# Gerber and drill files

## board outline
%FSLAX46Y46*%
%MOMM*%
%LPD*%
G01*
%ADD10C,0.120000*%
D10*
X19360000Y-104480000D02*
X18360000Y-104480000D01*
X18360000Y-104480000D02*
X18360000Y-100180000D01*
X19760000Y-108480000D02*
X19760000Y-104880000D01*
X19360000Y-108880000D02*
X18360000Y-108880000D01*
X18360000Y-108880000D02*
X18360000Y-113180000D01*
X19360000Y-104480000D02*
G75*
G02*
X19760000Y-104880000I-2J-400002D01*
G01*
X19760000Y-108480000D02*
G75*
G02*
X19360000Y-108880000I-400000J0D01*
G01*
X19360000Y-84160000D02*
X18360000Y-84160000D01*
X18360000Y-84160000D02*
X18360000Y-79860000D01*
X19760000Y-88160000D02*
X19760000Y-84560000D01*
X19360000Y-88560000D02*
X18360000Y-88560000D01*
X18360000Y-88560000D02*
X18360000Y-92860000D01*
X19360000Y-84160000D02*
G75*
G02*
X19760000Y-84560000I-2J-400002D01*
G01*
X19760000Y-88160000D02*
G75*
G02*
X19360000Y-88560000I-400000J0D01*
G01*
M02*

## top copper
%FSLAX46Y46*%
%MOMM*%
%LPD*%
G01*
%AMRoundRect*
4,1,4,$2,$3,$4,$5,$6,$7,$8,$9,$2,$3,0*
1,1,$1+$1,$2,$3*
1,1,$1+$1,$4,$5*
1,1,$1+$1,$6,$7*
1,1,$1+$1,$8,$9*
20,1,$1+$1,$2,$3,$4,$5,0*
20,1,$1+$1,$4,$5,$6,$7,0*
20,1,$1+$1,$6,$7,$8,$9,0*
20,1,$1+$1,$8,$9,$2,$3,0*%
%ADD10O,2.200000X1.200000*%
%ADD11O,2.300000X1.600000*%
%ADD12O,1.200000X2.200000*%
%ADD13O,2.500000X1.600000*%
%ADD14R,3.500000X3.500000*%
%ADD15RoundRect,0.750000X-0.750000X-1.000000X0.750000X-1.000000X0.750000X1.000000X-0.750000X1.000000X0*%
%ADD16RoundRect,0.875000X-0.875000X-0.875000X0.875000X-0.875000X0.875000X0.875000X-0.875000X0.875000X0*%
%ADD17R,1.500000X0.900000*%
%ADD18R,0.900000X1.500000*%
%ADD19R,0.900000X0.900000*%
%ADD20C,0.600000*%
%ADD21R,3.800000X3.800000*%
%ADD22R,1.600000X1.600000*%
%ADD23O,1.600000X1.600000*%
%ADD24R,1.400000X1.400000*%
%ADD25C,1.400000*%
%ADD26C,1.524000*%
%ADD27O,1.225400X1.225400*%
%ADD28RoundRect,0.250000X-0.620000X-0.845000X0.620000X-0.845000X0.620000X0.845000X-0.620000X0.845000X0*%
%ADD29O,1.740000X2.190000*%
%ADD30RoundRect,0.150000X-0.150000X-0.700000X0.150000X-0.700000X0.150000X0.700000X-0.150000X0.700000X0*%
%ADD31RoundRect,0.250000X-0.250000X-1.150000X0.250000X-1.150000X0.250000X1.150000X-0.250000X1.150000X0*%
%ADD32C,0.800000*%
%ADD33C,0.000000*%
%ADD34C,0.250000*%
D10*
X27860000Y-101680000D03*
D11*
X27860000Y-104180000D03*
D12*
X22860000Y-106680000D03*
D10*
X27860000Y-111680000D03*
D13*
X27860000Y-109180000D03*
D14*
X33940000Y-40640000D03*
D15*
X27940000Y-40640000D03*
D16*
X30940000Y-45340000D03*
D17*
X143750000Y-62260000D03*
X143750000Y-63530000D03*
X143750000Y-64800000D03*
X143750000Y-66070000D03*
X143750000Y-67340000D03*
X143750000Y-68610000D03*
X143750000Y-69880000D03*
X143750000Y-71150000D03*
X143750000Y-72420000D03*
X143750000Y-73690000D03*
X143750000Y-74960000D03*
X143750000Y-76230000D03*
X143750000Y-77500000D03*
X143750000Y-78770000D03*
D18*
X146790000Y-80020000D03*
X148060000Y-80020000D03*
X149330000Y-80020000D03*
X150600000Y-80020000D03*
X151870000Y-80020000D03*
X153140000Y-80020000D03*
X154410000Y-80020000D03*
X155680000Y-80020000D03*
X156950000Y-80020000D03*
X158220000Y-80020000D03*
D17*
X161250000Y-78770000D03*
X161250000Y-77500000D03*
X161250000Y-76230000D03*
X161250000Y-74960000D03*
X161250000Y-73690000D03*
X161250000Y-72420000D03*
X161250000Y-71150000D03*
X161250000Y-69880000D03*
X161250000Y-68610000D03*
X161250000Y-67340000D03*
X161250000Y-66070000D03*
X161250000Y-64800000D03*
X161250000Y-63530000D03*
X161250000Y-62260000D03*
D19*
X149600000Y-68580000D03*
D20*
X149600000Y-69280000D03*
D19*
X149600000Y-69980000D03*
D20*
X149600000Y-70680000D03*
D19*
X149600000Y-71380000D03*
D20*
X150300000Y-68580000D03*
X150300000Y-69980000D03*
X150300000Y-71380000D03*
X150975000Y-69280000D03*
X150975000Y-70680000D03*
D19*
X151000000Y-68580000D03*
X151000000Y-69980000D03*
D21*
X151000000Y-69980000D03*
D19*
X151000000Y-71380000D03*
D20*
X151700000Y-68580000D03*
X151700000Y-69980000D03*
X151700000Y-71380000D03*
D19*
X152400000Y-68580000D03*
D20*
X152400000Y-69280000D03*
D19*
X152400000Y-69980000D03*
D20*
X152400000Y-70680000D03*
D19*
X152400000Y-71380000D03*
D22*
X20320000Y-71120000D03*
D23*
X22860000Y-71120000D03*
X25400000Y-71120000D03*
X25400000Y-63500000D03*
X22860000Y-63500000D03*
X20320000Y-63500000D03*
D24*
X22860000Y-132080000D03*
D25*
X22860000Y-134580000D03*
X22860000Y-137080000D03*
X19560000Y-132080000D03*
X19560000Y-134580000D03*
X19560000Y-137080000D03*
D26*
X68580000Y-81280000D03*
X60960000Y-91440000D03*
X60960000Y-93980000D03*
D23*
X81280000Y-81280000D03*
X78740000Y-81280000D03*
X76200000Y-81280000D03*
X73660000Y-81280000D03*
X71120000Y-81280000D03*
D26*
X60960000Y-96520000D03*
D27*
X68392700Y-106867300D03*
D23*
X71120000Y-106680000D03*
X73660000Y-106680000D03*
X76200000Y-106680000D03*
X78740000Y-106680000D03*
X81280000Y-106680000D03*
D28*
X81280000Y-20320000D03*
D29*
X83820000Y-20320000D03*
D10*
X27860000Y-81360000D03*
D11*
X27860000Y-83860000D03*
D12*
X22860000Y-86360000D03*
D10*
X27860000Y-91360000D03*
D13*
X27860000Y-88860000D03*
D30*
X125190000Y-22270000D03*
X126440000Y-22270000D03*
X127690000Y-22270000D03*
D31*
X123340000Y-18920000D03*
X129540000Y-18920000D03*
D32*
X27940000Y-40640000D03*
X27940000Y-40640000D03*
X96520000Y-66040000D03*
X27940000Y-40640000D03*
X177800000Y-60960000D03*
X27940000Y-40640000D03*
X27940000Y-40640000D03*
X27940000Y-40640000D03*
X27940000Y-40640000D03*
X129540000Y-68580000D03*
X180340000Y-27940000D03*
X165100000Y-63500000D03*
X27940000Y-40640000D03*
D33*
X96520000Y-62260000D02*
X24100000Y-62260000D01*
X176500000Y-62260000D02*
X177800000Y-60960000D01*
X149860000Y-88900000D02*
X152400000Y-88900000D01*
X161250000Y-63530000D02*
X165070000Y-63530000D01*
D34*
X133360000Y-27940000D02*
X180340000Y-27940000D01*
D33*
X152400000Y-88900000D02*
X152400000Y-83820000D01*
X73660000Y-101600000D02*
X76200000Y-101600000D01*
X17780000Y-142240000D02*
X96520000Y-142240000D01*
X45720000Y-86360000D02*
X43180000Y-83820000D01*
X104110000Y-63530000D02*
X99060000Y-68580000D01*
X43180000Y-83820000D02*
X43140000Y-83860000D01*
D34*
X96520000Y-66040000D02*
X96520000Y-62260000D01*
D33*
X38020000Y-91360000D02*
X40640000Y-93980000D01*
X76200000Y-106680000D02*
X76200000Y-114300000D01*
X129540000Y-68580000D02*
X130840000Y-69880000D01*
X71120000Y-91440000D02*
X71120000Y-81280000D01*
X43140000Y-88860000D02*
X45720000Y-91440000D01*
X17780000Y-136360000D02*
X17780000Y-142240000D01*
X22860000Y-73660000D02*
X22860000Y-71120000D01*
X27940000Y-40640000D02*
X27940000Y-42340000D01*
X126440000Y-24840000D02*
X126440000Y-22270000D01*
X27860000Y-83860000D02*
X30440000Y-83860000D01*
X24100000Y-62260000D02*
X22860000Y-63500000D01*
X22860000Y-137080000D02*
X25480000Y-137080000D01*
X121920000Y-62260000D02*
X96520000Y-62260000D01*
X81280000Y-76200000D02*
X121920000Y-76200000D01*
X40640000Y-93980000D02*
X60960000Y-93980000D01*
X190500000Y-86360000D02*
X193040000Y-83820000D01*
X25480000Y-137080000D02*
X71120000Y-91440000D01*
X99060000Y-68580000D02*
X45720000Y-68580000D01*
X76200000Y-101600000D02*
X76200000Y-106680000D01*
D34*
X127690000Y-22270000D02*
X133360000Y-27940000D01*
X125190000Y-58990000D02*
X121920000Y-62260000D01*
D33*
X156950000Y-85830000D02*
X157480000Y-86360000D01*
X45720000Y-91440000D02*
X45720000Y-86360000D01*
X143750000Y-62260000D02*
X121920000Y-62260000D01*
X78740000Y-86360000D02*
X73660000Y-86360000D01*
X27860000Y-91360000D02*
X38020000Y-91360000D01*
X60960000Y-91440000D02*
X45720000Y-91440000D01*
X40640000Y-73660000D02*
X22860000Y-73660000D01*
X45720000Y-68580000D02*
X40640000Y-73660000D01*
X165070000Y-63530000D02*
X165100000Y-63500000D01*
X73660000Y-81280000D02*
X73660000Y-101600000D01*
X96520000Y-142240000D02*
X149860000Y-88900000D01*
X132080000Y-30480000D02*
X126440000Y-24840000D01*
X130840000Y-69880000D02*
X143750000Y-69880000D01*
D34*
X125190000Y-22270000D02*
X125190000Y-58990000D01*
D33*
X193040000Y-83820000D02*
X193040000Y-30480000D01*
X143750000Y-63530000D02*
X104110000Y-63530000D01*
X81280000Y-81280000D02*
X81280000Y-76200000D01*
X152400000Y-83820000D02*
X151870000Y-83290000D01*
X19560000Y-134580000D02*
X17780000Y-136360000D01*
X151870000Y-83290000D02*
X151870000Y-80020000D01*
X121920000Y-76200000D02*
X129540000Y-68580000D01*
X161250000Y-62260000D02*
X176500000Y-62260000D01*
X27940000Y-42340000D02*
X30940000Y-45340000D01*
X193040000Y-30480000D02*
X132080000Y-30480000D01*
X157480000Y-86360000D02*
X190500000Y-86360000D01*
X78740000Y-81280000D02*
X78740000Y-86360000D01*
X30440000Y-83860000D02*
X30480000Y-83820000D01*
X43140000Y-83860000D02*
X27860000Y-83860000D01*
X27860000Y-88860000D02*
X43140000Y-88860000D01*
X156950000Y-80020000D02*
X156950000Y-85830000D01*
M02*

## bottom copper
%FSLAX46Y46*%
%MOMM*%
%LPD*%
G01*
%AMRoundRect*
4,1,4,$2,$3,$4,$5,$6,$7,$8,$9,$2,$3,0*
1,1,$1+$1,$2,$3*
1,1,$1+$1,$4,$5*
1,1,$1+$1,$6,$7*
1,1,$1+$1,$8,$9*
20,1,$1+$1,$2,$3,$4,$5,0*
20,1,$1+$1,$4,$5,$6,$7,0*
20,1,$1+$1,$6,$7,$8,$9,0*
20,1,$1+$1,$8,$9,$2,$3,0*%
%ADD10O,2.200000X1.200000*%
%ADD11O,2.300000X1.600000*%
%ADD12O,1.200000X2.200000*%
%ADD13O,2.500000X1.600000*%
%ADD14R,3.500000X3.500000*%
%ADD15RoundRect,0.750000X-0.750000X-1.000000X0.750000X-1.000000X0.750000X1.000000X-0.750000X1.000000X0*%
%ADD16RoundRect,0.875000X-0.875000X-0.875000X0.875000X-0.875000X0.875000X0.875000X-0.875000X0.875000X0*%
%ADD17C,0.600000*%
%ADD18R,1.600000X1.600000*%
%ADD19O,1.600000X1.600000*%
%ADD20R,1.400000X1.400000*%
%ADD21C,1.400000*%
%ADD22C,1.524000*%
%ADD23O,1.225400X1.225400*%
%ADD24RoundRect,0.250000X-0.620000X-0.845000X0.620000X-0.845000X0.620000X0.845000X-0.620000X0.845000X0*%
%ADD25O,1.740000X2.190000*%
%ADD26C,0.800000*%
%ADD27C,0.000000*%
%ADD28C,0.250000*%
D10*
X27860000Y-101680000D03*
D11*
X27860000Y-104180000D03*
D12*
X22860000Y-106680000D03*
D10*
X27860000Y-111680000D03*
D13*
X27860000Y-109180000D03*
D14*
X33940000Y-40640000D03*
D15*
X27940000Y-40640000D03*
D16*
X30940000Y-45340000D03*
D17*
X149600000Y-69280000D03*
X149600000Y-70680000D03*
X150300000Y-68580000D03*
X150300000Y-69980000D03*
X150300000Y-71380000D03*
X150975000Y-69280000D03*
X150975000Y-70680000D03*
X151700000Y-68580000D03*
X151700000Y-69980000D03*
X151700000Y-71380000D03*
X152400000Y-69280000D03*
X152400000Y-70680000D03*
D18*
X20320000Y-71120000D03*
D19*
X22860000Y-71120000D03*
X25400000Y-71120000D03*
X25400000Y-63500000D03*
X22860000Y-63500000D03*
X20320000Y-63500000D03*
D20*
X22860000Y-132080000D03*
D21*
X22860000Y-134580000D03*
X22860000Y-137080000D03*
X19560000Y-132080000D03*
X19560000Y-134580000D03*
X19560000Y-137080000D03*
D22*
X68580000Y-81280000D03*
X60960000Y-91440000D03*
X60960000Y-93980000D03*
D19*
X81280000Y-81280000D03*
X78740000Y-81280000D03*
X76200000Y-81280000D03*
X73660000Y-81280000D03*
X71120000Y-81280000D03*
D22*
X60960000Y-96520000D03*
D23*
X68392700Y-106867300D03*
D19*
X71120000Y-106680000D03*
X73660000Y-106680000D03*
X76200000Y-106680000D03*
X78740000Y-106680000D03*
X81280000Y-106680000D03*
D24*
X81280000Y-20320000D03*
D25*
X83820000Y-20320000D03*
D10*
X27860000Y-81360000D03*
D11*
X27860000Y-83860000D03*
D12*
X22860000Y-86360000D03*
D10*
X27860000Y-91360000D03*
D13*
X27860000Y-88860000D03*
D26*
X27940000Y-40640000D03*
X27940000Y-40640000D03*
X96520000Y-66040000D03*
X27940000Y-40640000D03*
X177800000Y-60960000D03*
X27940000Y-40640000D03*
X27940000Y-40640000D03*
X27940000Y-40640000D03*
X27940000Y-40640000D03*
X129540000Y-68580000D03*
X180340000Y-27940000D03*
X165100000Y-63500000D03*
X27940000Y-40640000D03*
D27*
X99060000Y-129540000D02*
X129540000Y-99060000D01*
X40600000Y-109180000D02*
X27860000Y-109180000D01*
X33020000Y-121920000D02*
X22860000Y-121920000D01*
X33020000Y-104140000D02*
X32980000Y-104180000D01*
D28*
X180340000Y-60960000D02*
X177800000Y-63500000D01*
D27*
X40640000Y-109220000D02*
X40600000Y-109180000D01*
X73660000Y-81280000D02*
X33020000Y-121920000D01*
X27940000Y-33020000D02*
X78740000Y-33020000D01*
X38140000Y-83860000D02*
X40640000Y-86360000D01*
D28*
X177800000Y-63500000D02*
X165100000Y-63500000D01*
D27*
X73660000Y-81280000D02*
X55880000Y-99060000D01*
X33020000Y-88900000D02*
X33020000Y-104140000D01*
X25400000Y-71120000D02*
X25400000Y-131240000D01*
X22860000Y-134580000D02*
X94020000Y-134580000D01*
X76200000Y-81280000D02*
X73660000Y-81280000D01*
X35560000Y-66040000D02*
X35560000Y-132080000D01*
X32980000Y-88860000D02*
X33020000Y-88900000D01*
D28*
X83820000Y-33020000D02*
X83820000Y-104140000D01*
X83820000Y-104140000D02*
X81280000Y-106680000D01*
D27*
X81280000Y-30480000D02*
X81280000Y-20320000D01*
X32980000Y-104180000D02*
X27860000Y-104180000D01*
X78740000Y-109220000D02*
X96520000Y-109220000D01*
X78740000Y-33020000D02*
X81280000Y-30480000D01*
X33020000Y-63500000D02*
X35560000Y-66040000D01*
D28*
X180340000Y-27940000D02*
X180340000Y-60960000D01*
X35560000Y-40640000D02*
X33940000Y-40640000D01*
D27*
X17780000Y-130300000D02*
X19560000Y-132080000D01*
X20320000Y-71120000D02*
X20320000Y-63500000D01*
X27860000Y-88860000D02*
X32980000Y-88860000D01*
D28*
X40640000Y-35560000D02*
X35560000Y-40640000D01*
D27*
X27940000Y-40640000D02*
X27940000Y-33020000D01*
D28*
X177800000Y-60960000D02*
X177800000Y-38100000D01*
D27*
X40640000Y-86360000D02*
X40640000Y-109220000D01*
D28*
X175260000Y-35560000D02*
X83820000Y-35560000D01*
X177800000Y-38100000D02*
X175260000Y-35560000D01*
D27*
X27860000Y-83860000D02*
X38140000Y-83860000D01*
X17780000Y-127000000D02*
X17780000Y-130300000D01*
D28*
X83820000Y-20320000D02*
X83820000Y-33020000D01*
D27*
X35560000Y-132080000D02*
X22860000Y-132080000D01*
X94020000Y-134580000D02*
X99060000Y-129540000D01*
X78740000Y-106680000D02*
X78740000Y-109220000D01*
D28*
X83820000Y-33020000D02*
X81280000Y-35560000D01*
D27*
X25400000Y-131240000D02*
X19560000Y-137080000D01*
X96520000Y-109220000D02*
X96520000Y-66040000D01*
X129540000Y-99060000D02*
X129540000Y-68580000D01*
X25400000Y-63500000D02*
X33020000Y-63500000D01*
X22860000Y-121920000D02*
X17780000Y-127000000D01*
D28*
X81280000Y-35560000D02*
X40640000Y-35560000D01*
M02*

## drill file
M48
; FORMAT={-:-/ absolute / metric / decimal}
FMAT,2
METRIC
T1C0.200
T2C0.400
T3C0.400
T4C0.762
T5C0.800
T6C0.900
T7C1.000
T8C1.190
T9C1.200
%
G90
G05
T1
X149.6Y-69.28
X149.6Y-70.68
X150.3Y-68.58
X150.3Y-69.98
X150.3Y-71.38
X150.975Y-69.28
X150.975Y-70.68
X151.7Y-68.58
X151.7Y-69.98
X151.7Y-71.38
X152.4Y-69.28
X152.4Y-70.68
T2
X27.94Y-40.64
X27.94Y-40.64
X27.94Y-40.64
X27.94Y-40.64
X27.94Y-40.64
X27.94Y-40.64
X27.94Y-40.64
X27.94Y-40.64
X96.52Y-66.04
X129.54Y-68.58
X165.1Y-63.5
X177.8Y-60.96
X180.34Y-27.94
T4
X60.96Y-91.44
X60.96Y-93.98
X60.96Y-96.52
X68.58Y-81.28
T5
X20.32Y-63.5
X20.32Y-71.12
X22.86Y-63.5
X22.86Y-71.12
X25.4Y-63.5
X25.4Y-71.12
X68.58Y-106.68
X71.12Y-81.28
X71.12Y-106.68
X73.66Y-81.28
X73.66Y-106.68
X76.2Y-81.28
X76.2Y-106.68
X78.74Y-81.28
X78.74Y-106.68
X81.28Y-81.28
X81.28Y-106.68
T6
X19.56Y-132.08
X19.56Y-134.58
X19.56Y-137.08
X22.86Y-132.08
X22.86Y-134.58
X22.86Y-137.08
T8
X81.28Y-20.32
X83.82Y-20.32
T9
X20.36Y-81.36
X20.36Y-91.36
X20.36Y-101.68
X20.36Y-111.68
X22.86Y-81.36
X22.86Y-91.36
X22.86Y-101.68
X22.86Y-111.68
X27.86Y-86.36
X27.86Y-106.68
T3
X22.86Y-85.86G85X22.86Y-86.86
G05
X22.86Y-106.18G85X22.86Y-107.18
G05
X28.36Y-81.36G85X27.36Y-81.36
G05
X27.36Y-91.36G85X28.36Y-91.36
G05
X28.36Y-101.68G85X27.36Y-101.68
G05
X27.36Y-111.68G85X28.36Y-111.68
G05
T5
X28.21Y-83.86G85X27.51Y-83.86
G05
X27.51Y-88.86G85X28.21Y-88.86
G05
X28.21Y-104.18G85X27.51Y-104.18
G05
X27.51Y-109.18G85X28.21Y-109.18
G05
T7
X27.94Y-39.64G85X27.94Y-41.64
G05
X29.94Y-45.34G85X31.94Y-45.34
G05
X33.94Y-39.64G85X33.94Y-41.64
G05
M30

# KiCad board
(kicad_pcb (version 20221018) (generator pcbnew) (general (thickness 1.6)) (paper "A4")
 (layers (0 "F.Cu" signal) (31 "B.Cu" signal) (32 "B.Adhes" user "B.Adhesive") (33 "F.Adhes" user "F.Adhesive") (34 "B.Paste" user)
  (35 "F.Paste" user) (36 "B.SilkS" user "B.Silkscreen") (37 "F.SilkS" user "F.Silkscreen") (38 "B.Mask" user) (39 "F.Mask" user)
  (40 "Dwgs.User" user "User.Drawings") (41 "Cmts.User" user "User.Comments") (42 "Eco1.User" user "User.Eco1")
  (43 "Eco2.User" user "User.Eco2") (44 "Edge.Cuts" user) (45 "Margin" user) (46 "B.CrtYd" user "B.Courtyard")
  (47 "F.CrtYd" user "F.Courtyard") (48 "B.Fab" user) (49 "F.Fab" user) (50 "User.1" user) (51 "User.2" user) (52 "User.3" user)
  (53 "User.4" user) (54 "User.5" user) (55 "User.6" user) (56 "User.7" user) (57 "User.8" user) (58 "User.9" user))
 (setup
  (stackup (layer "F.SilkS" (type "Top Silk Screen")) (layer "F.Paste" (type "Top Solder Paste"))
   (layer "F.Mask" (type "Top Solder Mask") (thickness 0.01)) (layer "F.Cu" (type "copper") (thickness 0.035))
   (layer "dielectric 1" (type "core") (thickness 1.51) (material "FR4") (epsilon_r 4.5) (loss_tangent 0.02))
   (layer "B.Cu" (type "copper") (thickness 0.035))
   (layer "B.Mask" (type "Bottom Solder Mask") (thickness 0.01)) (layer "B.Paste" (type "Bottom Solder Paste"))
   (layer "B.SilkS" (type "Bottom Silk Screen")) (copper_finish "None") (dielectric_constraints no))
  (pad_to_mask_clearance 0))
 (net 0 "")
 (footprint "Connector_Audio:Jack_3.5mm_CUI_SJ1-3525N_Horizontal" (layer "F.Cu") (at 22.86 106.68 -90)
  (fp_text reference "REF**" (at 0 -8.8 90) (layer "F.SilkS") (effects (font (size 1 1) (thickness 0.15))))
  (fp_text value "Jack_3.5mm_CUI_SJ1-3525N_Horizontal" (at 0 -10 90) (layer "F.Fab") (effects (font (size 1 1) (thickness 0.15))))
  (fp_line (start -2.2 3.5) (end -2.2 4.5) (stroke (width 0.12) (type solid)) (layer "Edge.Cuts"))
  (fp_line (start -2.2 4.5) (end -6.5 4.5) (stroke (width 0.12) (type solid)) (layer "Edge.Cuts"))
  (fp_line (start 1.8 3.1) (end -1.8 3.1) (stroke (width 0.12) (type solid)) (layer "Edge.Cuts"))
  (fp_line (start 2.2 3.5) (end 2.2 4.5) (stroke (width 0.12) (type solid)) (layer "Edge.Cuts"))
  (fp_line (start 2.2 4.5) (end 6.5 4.5) (stroke (width 0.12) (type solid)) (layer "Edge.Cuts"))
  (fp_arc (start -2.2 3.5) (mid -2.082842 3.217158) (end -1.8 3.1) (stroke (width 0.12) (type solid)) (layer "Edge.Cuts"))
  (fp_arc (start 1.8 3.1) (mid 2.082843 3.217157) (end 2.2 3.5) (stroke (width 0.12) (type solid)) (layer "Edge.Cuts"))
  (pad "" np_thru_hole circle (at -5 0 270) (size 1.2 1.2) (drill 1.2) (layers "*.Cu"))
  (pad "" np_thru_hole circle (at -5 2.5 270) (size 1.2 1.2) (drill 1.2) (layers "*.Cu"))
  (pad "" np_thru_hole circle (at 0 -5 270) (size 1.2 1.2) (drill 1.2) (layers "*.Cu"))
  (pad "" np_thru_hole circle (at 5 0 270) (size 1.2 1.2) (drill 1.2) (layers "*.Cu"))
  (pad "" np_thru_hole circle (at 5 2.5 270) (size 1.2 1.2) (drill 1.2) (layers "*.Cu"))
  (pad "R" thru_hole oval (at -5 -5 270) (size 1.2 2.2) (drill oval 0.4 1.4) (layers "*.Cu" "*.Mask"))
  (pad "RN" thru_hole oval (at -2.5 -5 270) (size 1.6 2.3) (drill oval 0.8 1.5) (layers "*.Cu" "*.Mask"))
  (pad "S" thru_hole oval (at 0 0 270) (size 2.2 1.2) (drill oval 1.4 0.4) (layers "*.Cu" "*.Mask"))
  (pad "T" thru_hole oval (at 5 -5 90) (size 1.2 2.2) (drill oval 0.4 1.4) (layers "*.Cu" "*.Mask"))
  (pad "TN" thru_hole oval (at 2.5 -5 90) (size 1.6 2.5) (drill oval 0.8 1.5) (layers "*.Cu" "*.Mask")))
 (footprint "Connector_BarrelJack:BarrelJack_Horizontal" (layer "F.Cu") (at 33.94 40.64)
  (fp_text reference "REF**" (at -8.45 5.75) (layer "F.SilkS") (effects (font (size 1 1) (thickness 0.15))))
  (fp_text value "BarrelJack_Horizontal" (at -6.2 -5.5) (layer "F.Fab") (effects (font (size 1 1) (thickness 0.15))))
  (pad "1" thru_hole rect (at 0 0) (size 3.5 3.5) (drill oval 1 3) (layers "*.Cu" "*.Mask"))
  (pad "2" thru_hole roundrect (at -6 0) (size 3 3.5) (drill oval 1 3) (layers "*.Cu" "*.Mask") (roundrect_rratio 0.25))
  (pad "3" thru_hole roundrect (at -3 4.7) (size 3.5 3.5) (drill oval 3 1) (layers "*.Cu" "*.Mask") (roundrect_rratio 0.25)))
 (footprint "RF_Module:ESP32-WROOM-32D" (layer "F.Cu") (at 152.5 70.51)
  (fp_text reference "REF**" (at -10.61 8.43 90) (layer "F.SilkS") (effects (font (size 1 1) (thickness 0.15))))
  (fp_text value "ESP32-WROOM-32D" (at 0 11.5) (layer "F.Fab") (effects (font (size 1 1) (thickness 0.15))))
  (pad "1" smd rect (at -8.75 -8.25) (size 1.5 0.9) (layers "F.Cu" "F.Paste" "F.Mask"))
  (pad "2" smd rect (at -8.75 -6.98) (size 1.5 0.9) (layers "F.Cu" "F.Paste" "F.Mask"))
  (pad "3" smd rect (at -8.75 -5.71) (size 1.5 0.9) (layers "F.Cu" "F.Paste" "F.Mask"))
  (pad "4" smd rect (at -8.75 -4.44) (size 1.5 0.9) (layers "F.Cu" "F.Paste" "F.Mask"))
  (pad "5" smd rect (at -8.75 -3.17) (size 1.5 0.9) (layers "F.Cu" "F.Paste" "F.Mask"))
  (pad "6" smd rect (at -8.75 -1.9) (size 1.5 0.9) (layers "F.Cu" "F.Paste" "F.Mask"))
  (pad "7" smd rect (at -8.75 -0.63) (size 1.5 0.9) (layers "F.Cu" "F.Paste" "F.Mask"))
  (pad "8" smd rect (at -8.75 0.64) (size 1.5 0.9) (layers "F.Cu" "F.Paste" "F.Mask"))
  (pad "9" smd rect (at -8.75 1.91) (size 1.5 0.9) (layers "F.Cu" "F.Paste" "F.Mask"))
  (pad "10" smd rect (at -8.75 3.18) (size 1.5 0.9) (layers "F.Cu" "F.Paste" "F.Mask"))
  (pad "11" smd rect (at -8.75 4.45) (size 1.5 0.9) (layers "F.Cu" "F.Paste" "F.Mask"))
  (pad "12" smd rect (at -8.75 5.72) (size 1.5 0.9) (layers "F.Cu" "F.Paste" "F.Mask"))
  (pad "13" smd rect (at -8.75 6.99) (size 1.5 0.9) (layers "F.Cu" "F.Paste" "F.Mask"))
  (pad "14" smd rect (at -8.75 8.26) (size 1.5 0.9) (layers "F.Cu" "F.Paste" "F.Mask"))
  (pad "15" smd rect (at -5.71 9.51 90) (size 1.5 0.9) (layers "F.Cu" "F.Paste" "F.Mask"))
  (pad "16" smd rect (at -4.44 9.51 90) (size 1.5 0.9) (layers "F.Cu" "F.Paste" "F.Mask"))
  (pad "17" smd rect (at -3.17 9.51 90) (size 1.5 0.9) (layers "F.Cu" "F.Paste" "F.Mask"))
  (pad "18" smd rect (at -1.9 9.51 90) (size 1.5 0.9) (layers "F.Cu" "F.Paste" "F.Mask"))
  (pad "19" smd rect (at -0.63 9.51 90) (size 1.5 0.9) (layers "F.Cu" "F.Paste" "F.Mask"))
  (pad "20" smd rect (at 0.64 9.51 90) (size 1.5 0.9) (layers "F.Cu" "F.Paste" "F.Mask"))
  (pad "21" smd rect (at 1.91 9.51 90) (size 1.5 0.9) (layers "F.Cu" "F.Paste" "F.Mask"))
  (pad "22" smd rect (at 3.18 9.51 90) (size 1.5 0.9) (layers "F.Cu" "F.Paste" "F.Mask"))
  (pad "23" smd rect (at 4.45 9.51 90) (size 1.5 0.9) (layers "F.Cu" "F.Paste" "F.Mask"))
  (pad "24" smd rect (at 5.72 9.51 90) (size 1.5 0.9) (layers "F.Cu" "F.Paste" "F.Mask"))
  (pad "25" smd rect (at 8.75 8.26) (size 1.5 0.9) (layers "F.Cu" "F.Paste" "F.Mask"))
  (pad "26" smd rect (at 8.75 6.99) (size 1.5 0.9) (layers "F.Cu" "F.Paste" "F.Mask"))
  (pad "27" smd rect (at 8.75 5.72) (size 1.5 0.9) (layers "F.Cu" "F.Paste" "F.Mask"))
  (pad "28" smd rect (at 8.75 4.45) (size 1.5 0.9) (layers "F.Cu" "F.Paste" "F.Mask"))
  (pad "29" smd rect (at 8.75 3.18) (size 1.5 0.9) (layers "F.Cu" "F.Paste" "F.Mask"))
  (pad "30" smd rect (at 8.75 1.91) (size 1.5 0.9) (layers "F.Cu" "F.Paste" "F.Mask"))
  (pad "31" smd rect (at 8.75 0.64) (size 1.5 0.9) (layers "F.Cu" "F.Paste" "F.Mask"))
  (pad "32" smd rect (at 8.75 -0.63) (size 1.5 0.9) (layers "F.Cu" "F.Paste" "F.Mask"))
  (pad "33" smd rect (at 8.75 -1.9) (size 1.5 0.9) (layers "F.Cu" "F.Paste" "F.Mask"))
  (pad "34" smd rect (at 8.75 -3.17) (size 1.5 0.9) (layers "F.Cu" "F.Paste" "F.Mask"))
  (pad "35" smd rect (at 8.75 -4.44) (size 1.5 0.9) (layers "F.Cu" "F.Paste" "F.Mask"))
  (pad "36" smd rect (at 8.75 -5.71) (size 1.5 0.9) (layers "F.Cu" "F.Paste" "F.Mask"))
  (pad "37" smd rect (at 8.75 -6.98) (size 1.5 0.9) (layers "F.Cu" "F.Paste" "F.Mask"))
  (pad "38" smd rect (at 8.75 -8.25) (size 1.5 0.9) (layers "F.Cu" "F.Paste" "F.Mask"))
  (pad "39" smd rect (at -2.9 -1.93) (size 0.9 0.9) (layers "F.Cu" "F.Paste"))
  (pad "39" thru_hole circle (at -2.9 -1.23) (size 0.6 0.6) (drill 0.2) (layers "*.Cu" "F.Mask"))
  (pad "39" smd rect (at -2.9 -0.53) (size 0.9 0.9) (layers "F.Cu" "F.Paste"))
  (pad "39" thru_hole circle (at -2.9 0.17) (size 0.6 0.6) (drill 0.2) (layers "*.Cu" "F.Mask"))
  (pad "39" smd rect (at -2.9 0.87) (size 0.9 0.9) (layers "F.Cu" "F.Paste"))
  (pad "39" thru_hole circle (at -2.2 -1.93) (size 0.6 0.6) (drill 0.2) (layers "*.Cu" "F.Mask"))
  (pad "39" thru_hole circle (at -2.2 -0.53) (size 0.6 0.6) (drill 0.2) (layers "*.Cu" "F.Mask"))
  (pad "39" thru_hole circle (at -2.2 0.87) (size 0.6 0.6) (drill 0.2) (layers "*.Cu" "F.Mask"))
  (pad "39" thru_hole circle (at -1.525 -1.23) (size 0.6 0.6) (drill 0.2) (layers "*.Cu" "F.Mask"))
  (pad "39" thru_hole circle (at -1.525 0.17) (size 0.6 0.6) (drill 0.2) (layers "*.Cu" "F.Mask"))
  (pad "39" smd rect (at -1.5 -1.93) (size 0.9 0.9) (layers "F.Cu" "F.Paste"))
  (pad "39" smd rect (at -1.5 -0.53) (size 0.9 0.9) (layers "F.Cu" "F.Paste"))
  (pad "39" smd rect (at -1.5 -0.53) (size 3.8 3.8) (layers "F.Cu" "F.Mask"))
  (pad "39" smd rect (at -1.5 0.87) (size 0.9 0.9) (layers "F.Cu" "F.Paste"))
  (pad "39" thru_hole circle (at -0.8 -1.93) (size 0.6 0.6) (drill 0.2) (layers "*.Cu" "F.Mask"))
  (pad "39" thru_hole circle (at -0.8 -0.53) (size 0.6 0.6) (drill 0.2) (layers "*.Cu" "F.Mask"))
  (pad "39" thru_hole circle (at -0.8 0.87) (size 0.6 0.6) (drill 0.2) (layers "*.Cu" "F.Mask"))
  (pad "39" smd rect (at -0.1 -1.93) (size 0.9 0.9) (layers "F.Cu" "F.Paste"))
  (pad "39" thru_hole circle (at -0.1 -1.23) (size 0.6 0.6) (drill 0.2) (layers "*.Cu" "F.Mask"))
  (pad "39" smd rect (at -0.1 -0.53) (size 0.9 0.9) (layers "F.Cu" "F.Paste"))
  (pad "39" thru_hole circle (at -0.1 0.17) (size 0.6 0.6) (drill 0.2) (layers "*.Cu" "F.Mask"))
  (pad "39" smd rect (at -0.1 0.87) (size 0.9 0.9) (layers "F.Cu" "F.Paste"))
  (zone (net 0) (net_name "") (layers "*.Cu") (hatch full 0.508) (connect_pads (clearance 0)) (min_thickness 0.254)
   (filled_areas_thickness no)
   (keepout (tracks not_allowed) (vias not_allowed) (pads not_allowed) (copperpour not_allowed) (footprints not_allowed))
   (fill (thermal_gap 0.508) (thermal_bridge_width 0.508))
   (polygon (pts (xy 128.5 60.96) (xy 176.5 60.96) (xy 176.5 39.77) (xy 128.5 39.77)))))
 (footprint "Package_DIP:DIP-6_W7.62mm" (layer "F.Cu") (at 20.32 71.12 90)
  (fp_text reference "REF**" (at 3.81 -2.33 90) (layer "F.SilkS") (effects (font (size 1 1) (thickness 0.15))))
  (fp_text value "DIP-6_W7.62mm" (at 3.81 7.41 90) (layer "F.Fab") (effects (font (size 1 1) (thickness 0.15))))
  (pad "1" thru_hole rect (at 0 0 90) (size 1.6 1.6) (drill 0.8) (layers "*.Cu" "*.Mask"))
  (pad "2" thru_hole oval (at 0 2.54 90) (size 1.6 1.6) (drill 0.8) (layers "*.Cu" "*.Mask"))
  (pad "3" thru_hole oval (at 0 5.08 90) (size 1.6 1.6) (drill 0.8) (layers "*.Cu" "*.Mask"))
  (pad "4" thru_hole oval (at 7.62 5.08 90) (size 1.6 1.6) (drill 0.8) (layers "*.Cu" "*.Mask"))
  (pad "5" thru_hole oval (at 7.62 2.54 90) (size 1.6 1.6) (drill 0.8) (layers "*.Cu" "*.Mask"))
  (pad "6" thru_hole oval (at 7.62 0 90) (size 1.6 1.6) (drill 0.8) (layers "*.Cu" "*.Mask")))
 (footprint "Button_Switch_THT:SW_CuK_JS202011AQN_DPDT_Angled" (layer "F.Cu") (at 22.86 132.08 -90)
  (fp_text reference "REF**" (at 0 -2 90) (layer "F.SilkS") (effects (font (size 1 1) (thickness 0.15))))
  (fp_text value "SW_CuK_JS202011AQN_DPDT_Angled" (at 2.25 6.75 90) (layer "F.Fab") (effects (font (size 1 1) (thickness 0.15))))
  (pad "1" thru_hole rect (at 0 0 270) (size 1.4 1.4) (drill 0.9) (layers "*.Cu" "*.Mask"))
  (pad "2" thru_hole circle (at 2.5 0 270) (size 1.4 1.4) (drill 0.9) (layers "*.Cu" "*.Mask"))
  (pad "3" thru_hole circle (at 5 0 270) (size 1.4 1.4) (drill 0.9) (layers "*.Cu" "*.Mask"))
  (pad "4" thru_hole circle (at 0 3.3 270) (size 1.4 1.4) (drill 0.9) (layers "*.Cu" "*.Mask"))
  (pad "5" thru_hole circle (at 2.5 3.3 270) (size 1.4 1.4) (drill 0.9) (layers "*.Cu" "*.Mask"))
  (pad "6" thru_hole circle (at 5 3.3 270) (size 1.4 1.4) (drill 0.9) (layers "*.Cu" "*.Mask")))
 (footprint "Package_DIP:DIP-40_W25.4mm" (layer "F.Cu") (at 88.9 81.28 -90)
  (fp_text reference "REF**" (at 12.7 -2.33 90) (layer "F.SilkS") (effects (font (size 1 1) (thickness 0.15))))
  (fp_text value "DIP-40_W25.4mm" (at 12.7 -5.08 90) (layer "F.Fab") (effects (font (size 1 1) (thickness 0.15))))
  (pad "1" thru_hole circle (at 0 20.32 270) (size 1.524 1.524) (drill 0.762) (layers "*.Cu" "*.Mask"))
  (pad "2" thru_hole circle (at 10.16 27.94 270) (size 1.524 1.524) (drill 0.762) (layers "*.Cu" "*.Mask"))
  (pad "3" thru_hole circle (at 12.7 27.94 270) (size 1.524 1.524) (drill 0.762) (layers "*.Cu" "*.Mask"))
  (pad "4" thru_hole oval (at 0 7.62 270) (size 1.6 1.6) (drill 0.8) (layers "*.Cu" "*.Mask"))
  (pad "5" thru_hole oval (at 0 10.16 270) (size 1.6 1.6) (drill 0.8) (layers "*.Cu" "*.Mask"))
  (pad "6" thru_hole oval (at 0 12.7 270) (size 1.6 1.6) (drill 0.8) (layers "*.Cu" "*.Mask"))
  (pad "7" thru_hole oval (at 0 15.24 270) (size 1.6 1.6) (drill 0.8) (layers "*.Cu" "*.Mask"))
  (pad "8" thru_hole oval (at 0 17.78 270) (size 1.6 1.6) (drill 0.8) (layers "*.Cu" "*.Mask"))
  (pad "11" thru_hole circle (at 15.24 27.94 270) (size 1.524 1.524) (drill 0.762) (layers "*.Cu" "*.Mask"))
  (pad "32" thru_hole oval (at 25.4 20.32 270) (size 1.2254 1.2254) (drill 0.8 (offset 0.1873 0.1873)) (layers "*.Cu" "*.Mask"))
  (pad "33" thru_hole oval (at 25.4 17.78 270) (size 1.6 1.6) (drill 0.8) (layers "*.Cu" "*.Mask"))
  (pad "34" thru_hole oval (at 25.4 15.24 270) (size 1.6 1.6) (drill 0.8) (layers "*.Cu" "*.Mask"))
  (pad "35" thru_hole oval (at 25.4 12.7 270) (size 1.6 1.6) (drill 0.8) (layers "*.Cu" "*.Mask"))
  (pad "36" thru_hole oval (at 25.4 10.16 270) (size 1.6 1.6) (drill 0.8) (layers "*.Cu" "*.Mask"))
  (pad "37" thru_hole oval (at 25.4 7.62 270) (size 1.6 1.6) (drill 0.8) (layers "*.Cu" "*.Mask")))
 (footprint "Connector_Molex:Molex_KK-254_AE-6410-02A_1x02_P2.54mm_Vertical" (layer "F.Cu") (at 81.28 20.32)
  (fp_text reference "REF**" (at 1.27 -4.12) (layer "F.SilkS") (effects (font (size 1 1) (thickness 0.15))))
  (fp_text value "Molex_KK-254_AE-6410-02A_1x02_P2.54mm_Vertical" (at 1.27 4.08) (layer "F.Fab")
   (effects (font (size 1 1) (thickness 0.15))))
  (pad "1" thru_hole roundrect (at 0 0) (size 1.74 2.19) (drill 1.19) (layers "*.Cu" "*.Mask") (roundrect_rratio 0.143678))
  (pad "2" thru_hole oval (at 2.54 0) (size 1.74 2.19) (drill 1.19) (layers "*.Cu" "*.Mask")))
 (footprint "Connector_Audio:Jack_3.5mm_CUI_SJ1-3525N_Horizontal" (layer "F.Cu") (at 22.86 86.36 -90)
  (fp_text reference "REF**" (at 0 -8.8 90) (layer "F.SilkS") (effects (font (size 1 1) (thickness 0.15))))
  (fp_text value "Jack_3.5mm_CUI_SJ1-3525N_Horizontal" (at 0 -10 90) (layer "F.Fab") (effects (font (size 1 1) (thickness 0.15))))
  (fp_line (start -2.2 3.5) (end -2.2 4.5) (stroke (width 0.12) (type solid)) (layer "Edge.Cuts"))
  (fp_line (start -2.2 4.5) (end -6.5 4.5) (stroke (width 0.12) (type solid)) (layer "Edge.Cuts"))
  (fp_line (start 1.8 3.1) (end -1.8 3.1) (stroke (width 0.12) (type solid)) (layer "Edge.Cuts"))
  (fp_line (start 2.2 3.5) (end 2.2 4.5) (stroke (width 0.12) (type solid)) (layer "Edge.Cuts"))
  (fp_line (start 2.2 4.5) (end 6.5 4.5) (stroke (width 0.12) (type solid)) (layer "Edge.Cuts"))
  (fp_arc (start -2.2 3.5) (mid -2.082842 3.217158) (end -1.8 3.1) (stroke (width 0.12) (type solid)) (layer "Edge.Cuts"))
  (fp_arc (start 1.8 3.1) (mid 2.082843 3.217157) (end 2.2 3.5) (stroke (width 0.12) (type solid)) (layer "Edge.Cuts"))
  (pad "" np_thru_hole circle (at -5 0 270) (size 1.2 1.2) (drill 1.2) (layers "*.Cu"))
  (pad "" np_thru_hole circle (at -5 2.5 270) (size 1.2 1.2) (drill 1.2) (layers "*.Cu"))
  (pad "" np_thru_hole circle (at 0 -5 270) (size 1.2 1.2) (drill 1.2) (layers "*.Cu"))
  (pad "" np_thru_hole circle (at 5 0 270) (size 1.2 1.2) (drill 1.2) (layers "*.Cu"))
  (pad "" np_thru_hole circle (at 5 2.5 270) (size 1.2 1.2) (drill 1.2) (layers "*.Cu"))
  (pad "R" thru_hole oval (at -5 -5 270) (size 1.2 2.2) (drill oval 0.4 1.4) (layers "*.Cu" "*.Mask"))
  (pad "RN" thru_hole oval (at -2.5 -5 270) (size 1.6 2.3) (drill oval 0.8 1.5) (layers "*.Cu" "*.Mask"))
  (pad "S" thru_hole oval (at 0 0 270) (size 2.2 1.2) (drill oval 1.4 0.4) (layers "*.Cu" "*.Mask"))
  (pad "T" thru_hole oval (at 5 -5 90) (size 1.2 2.2) (drill oval 0.4 1.4) (layers "*.Cu" "*.Mask"))
  (pad "TN" thru_hole oval (at 2.5 -5 90) (size 1.6 2.5) (drill oval 0.8 1.5) (layers "*.Cu" "*.Mask")))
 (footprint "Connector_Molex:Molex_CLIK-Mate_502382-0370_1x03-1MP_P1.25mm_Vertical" (layer "F.Cu") (at 126.44 20.32)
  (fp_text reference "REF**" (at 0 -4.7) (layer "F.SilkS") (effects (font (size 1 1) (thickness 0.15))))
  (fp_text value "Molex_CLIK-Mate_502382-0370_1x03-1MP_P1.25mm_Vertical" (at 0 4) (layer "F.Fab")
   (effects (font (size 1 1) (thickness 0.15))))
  (pad "1" smd roundrect (at -1.25 1.95) (size 0.6 1.7) (layers "F.Cu" "F.Paste" "F.Mask") (roundrect_rratio 0.25))
  (pad "2" smd roundrect (at 0 1.95) (size 0.6 1.7) (layers "F.Cu" "F.Paste" "F.Mask") (roundrect_rratio 0.25))
  (pad "3" smd roundrect (at 1.25 1.95) (size 0.6 1.7) (layers "F.Cu" "F.Paste" "F.Mask") (roundrect_rratio 0.25))
  (pad "MP" smd roundrect (at -3.1 -1.4) (size 1 2.8) (layers "F.Cu" "F.Paste" "F.Mask") (roundrect_rratio 0.25))
  (pad "MP" smd roundrect (at 3.1 -1.4) (size 1 2.8) (layers "F.Cu" "F.Paste" "F.Mask") (roundrect_rratio 0.25)))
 (segment (start 96.52 62.26) (end 24.1 62.26) (width 0) (layer "F.Cu") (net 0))
 (segment (start 176.5 62.26) (end 177.8 60.96) (width 0) (layer "F.Cu") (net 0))
 (segment (start 149.86 88.9) (end 152.4 88.9) (width 0) (layer "F.Cu") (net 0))
 (segment (start 161.25 63.53) (end 165.07 63.53) (width 0) (layer "F.Cu") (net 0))
 (segment (start 133.36 27.94) (end 180.34 27.94) (width 0.25) (layer "F.Cu") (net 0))
 (segment (start 152.4 88.9) (end 152.4 83.82) (width 0) (layer "F.Cu") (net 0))
 (segment (start 73.66 101.6) (end 76.2 101.6) (width 0) (layer "F.Cu") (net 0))
 (segment (start 17.78 142.24) (end 96.52 142.24) (width 0) (layer "F.Cu") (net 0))
 (segment (start 45.72 86.36) (end 43.18 83.82) (width 0) (layer "F.Cu") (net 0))
 (segment (start 104.11 63.53) (end 99.06 68.58) (width 0) (layer "F.Cu") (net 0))
 (segment (start 43.18 83.82) (end 43.14 83.86) (width 0) (layer "F.Cu") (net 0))
 (segment (start 96.52 66.04) (end 96.52 62.26) (width 0.25) (layer "F.Cu") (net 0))
 (segment (start 38.02 91.36) (end 40.64 93.98) (width 0) (layer "F.Cu") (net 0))
 (segment (start 76.2 106.68) (end 76.2 114.3) (width 0) (layer "F.Cu") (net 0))
 (segment (start 129.54 68.58) (end 130.84 69.88) (width 0) (layer "F.Cu") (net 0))
 (segment (start 71.12 91.44) (end 71.12 81.28) (width 0) (layer "F.Cu") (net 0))
 (segment (start 43.14 88.86) (end 45.72 91.44) (width 0) (layer "F.Cu") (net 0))
 (segment (start 17.78 136.36) (end 17.78 142.24) (width 0) (layer "F.Cu") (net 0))
 (segment (start 22.86 73.66) (end 22.86 71.12) (width 0) (layer "F.Cu") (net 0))
 (segment (start 27.94 40.64) (end 27.94 42.34) (width 0) (layer "F.Cu") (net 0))
 (segment (start 126.44 24.84) (end 126.44 22.27) (width 0) (layer "F.Cu") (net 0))
 (segment (start 27.86 83.86) (end 30.44 83.86) (width 0) (layer "F.Cu") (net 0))
 (segment (start 24.1 62.26) (end 22.86 63.5) (width 0) (layer "F.Cu") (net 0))
 (segment (start 22.86 137.08) (end 25.48 137.08) (width 0) (layer "F.Cu") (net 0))
 (segment (start 121.92 62.26) (end 96.52 62.26) (width 0) (layer "F.Cu") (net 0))
 (segment (start 81.28 76.2) (end 121.92 76.2) (width 0) (layer "F.Cu") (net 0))
 (segment (start 40.64 93.98) (end 60.96 93.98) (width 0) (layer "F.Cu") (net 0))
 (segment (start 190.5 86.36) (end 193.04 83.82) (width 0) (layer "F.Cu") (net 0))
 (segment (start 25.48 137.08) (end 71.12 91.44) (width 0) (layer "F.Cu") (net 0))
 (segment (start 99.06 68.58) (end 45.72 68.58) (width 0) (layer "F.Cu") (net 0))
 (segment (start 76.2 101.6) (end 76.2 106.68) (width 0) (layer "F.Cu") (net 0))
 (segment (start 127.69 22.27) (end 133.36 27.94) (width 0.25) (layer "F.Cu") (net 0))
 (segment (start 125.19 58.99) (end 121.92 62.26) (width 0.25) (layer "F.Cu") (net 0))
 (segment (start 156.95 85.83) (end 157.48 86.36) (width 0) (layer "F.Cu") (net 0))
 (segment (start 45.72 91.44) (end 45.72 86.36) (width 0) (layer "F.Cu") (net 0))
 (segment (start 143.75 62.26) (end 121.92 62.26) (width 0) (layer "F.Cu") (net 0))
 (segment (start 78.74 86.36) (end 73.66 86.36) (width 0) (layer "F.Cu") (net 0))
 (segment (start 27.86 91.36) (end 38.02 91.36) (width 0) (layer "F.Cu") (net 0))
 (segment (start 60.96 91.44) (end 45.72 91.44) (width 0) (layer "F.Cu") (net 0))
 (segment (start 40.64 73.66) (end 22.86 73.66) (width 0) (layer "F.Cu") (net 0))
 (segment (start 45.72 68.58) (end 40.64 73.66) (width 0) (layer "F.Cu") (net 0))
 (segment (start 165.07 63.53) (end 165.1 63.5) (width 0) (layer "F.Cu") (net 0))
 (segment (start 73.66 81.28) (end 73.66 101.6) (width 0) (layer "F.Cu") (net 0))
 (segment (start 96.52 142.24) (end 149.86 88.9) (width 0) (layer "F.Cu") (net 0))
 (segment (start 132.08 30.48) (end 126.44 24.84) (width 0) (layer "F.Cu") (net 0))
 (segment (start 130.84 69.88) (end 143.75 69.88) (width 0) (layer "F.Cu") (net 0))
 (segment (start 125.19 22.27) (end 125.19 58.99) (width 0.25) (layer "F.Cu") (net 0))
 (segment (start 193.04 83.82) (end 193.04 30.48) (width 0) (layer "F.Cu") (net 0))
 (segment (start 143.75 63.53) (end 104.11 63.53) (width 0) (layer "F.Cu") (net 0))
 (segment (start 81.28 81.28) (end 81.28 76.2) (width 0) (layer "F.Cu") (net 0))
 (segment (start 152.4 83.82) (end 151.87 83.29) (width 0) (layer "F.Cu") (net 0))
 (segment (start 19.56 134.58) (end 17.78 136.36) (width 0) (layer "F.Cu") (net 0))
 (segment (start 151.87 83.29) (end 151.87 80.02) (width 0) (layer "F.Cu") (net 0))
 (segment (start 121.92 76.2) (end 129.54 68.58) (width 0) (layer "F.Cu") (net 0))
 (segment (start 161.25 62.26) (end 176.5 62.26) (width 0) (layer "F.Cu") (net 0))
 (segment (start 27.94 42.34) (end 30.94 45.34) (width 0) (layer "F.Cu") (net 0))
 (segment (start 193.04 30.48) (end 132.08 30.48) (width 0) (layer "F.Cu") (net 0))
 (segment (start 157.48 86.36) (end 190.5 86.36) (width 0) (layer "F.Cu") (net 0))
 (segment (start 78.74 81.28) (end 78.74 86.36) (width 0) (layer "F.Cu") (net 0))
 (segment (start 30.44 83.86) (end 30.48 83.82) (width 0) (layer "F.Cu") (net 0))
 (segment (start 43.14 83.86) (end 27.86 83.86) (width 0) (layer "F.Cu") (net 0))
 (segment (start 27.86 88.86) (end 43.14 88.86) (width 0) (layer "F.Cu") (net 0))
 (segment (start 156.95 80.02) (end 156.95 85.83) (width 0) (layer "F.Cu") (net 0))
 (via (at 27.94 40.64) (size 0.8) (drill 0.4) (layers "F.Cu" "B.Cu") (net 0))
 (via (at 27.94 40.64) (size 0.8) (drill 0.4) (layers "F.Cu" "B.Cu") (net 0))
 (via (at 96.52 66.04) (size 0.8) (drill 0.4) (layers "F.Cu" "B.Cu") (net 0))
 (via (at 27.94 40.64) (size 0.8) (drill 0.4) (layers "F.Cu" "B.Cu") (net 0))
 (via (at 177.8 60.96) (size 0.8) (drill 0.4) (layers "F.Cu" "B.Cu") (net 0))
 (via (at 27.94 40.64) (size 0.8) (drill 0.4) (layers "F.Cu" "B.Cu") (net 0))
 (via (at 27.94 40.64) (size 0.8) (drill 0.4) (layers "F.Cu" "B.Cu") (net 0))
 (via (at 27.94 40.64) (size 0.8) (drill 0.4) (layers "F.Cu" "B.Cu") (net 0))
 (via (at 27.94 40.64) (size 0.8) (drill 0.4) (layers "F.Cu" "B.Cu") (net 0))
 (via (at 129.54 68.58) (size 0.8) (drill 0.4) (layers "F.Cu" "B.Cu") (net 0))
 (via (at 180.34 27.94) (size 0.8) (drill 0.4) (layers "F.Cu" "B.Cu") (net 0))
 (via (at 165.1 63.5) (size 0.8) (drill 0.4) (layers "F.Cu" "B.Cu") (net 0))
 (via (at 27.94 40.64) (size 0.8) (drill 0.4) (layers "F.Cu" "B.Cu") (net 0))
 (segment (start 99.06 129.54) (end 129.54 99.06) (width 0) (layer "B.Cu") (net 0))
 (segment (start 40.6 109.18) (end 27.86 109.18) (width 0) (layer "B.Cu") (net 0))
 (segment (start 33.02 121.92) (end 22.86 121.92) (width 0) (layer "B.Cu") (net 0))
 (segment (start 33.02 104.14) (end 32.98 104.18) (width 0) (layer "B.Cu") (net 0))
 (segment (start 180.34 60.96) (end 177.8 63.5) (width 0.25) (layer "B.Cu") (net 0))
 (segment (start 40.64 109.22) (end 40.6 109.18) (width 0) (layer "B.Cu") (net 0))
 (segment (start 73.66 81.28) (end 33.02 121.92) (width 0) (layer "B.Cu") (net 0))
 (segment (start 27.94 33.02) (end 78.74 33.02) (width 0) (layer "B.Cu") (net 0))
 (segment (start 38.14 83.86) (end 40.64 86.36) (width 0) (layer "B.Cu") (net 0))
 (segment (start 177.8 63.5) (end 165.1 63.5) (width 0.25) (layer "B.Cu") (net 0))
 (segment (start 73.66 81.28) (end 55.88 99.06) (width 0) (layer "B.Cu") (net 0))
 (segment (start 33.02 88.9) (end 33.02 104.14) (width 0) (layer "B.Cu") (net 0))
 (segment (start 25.4 71.12) (end 25.4 131.24) (width 0) (layer "B.Cu") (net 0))
 (segment (start 22.86 134.58) (end 94.02 134.58) (width 0) (layer "B.Cu") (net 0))
 (segment (start 76.2 81.28) (end 73.66 81.28) (width 0) (layer "B.Cu") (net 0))
 (segment (start 35.56 66.04) (end 35.56 132.08) (width 0) (layer "B.Cu") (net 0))
 (segment (start 32.98 88.86) (end 33.02 88.9) (width 0) (layer "B.Cu") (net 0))
 (segment (start 83.82 33.02) (end 83.82 104.14) (width 0.25) (layer "B.Cu") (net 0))
 (segment (start 83.82 104.14) (end 81.28 106.68) (width 0.25) (layer "B.Cu") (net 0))
 (segment (start 81.28 30.48) (end 81.28 20.32) (width 0) (layer "B.Cu") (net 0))
 (segment (start 32.98 104.18) (end 27.86 104.18) (width 0) (layer "B.Cu") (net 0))
 (segment (start 78.74 109.22) (end 96.52 109.22) (width 0) (layer "B.Cu") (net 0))
 (segment (start 78.74 33.02) (end 81.28 30.48) (width 0) (layer "B.Cu") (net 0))
 (segment (start 33.02 63.5) (end 35.56 66.04) (width 0) (layer "B.Cu") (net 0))
 (segment (start 180.34 27.94) (end 180.34 60.96) (width 0.25) (layer "B.Cu") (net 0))
 (segment (start 35.56 40.64) (end 33.94 40.64) (width 0.25) (layer "B.Cu") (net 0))
 (segment (start 17.78 130.3) (end 19.56 132.08) (width 0) (layer "B.Cu") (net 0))
 (segment (start 20.32 71.12) (end 20.32 63.5) (width 0) (layer "B.Cu") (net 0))
 (segment (start 27.86 88.86) (end 32.98 88.86) (width 0) (layer "B.Cu") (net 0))
 (segment (start 40.64 35.56) (end 35.56 40.64) (width 0.25) (layer "B.Cu") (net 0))
 (segment (start 27.94 40.64) (end 27.94 33.02) (width 0) (layer "B.Cu") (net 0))
 (segment (start 177.8 60.96) (end 177.8 38.1) (width 0.25) (layer "B.Cu") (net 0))
 (segment (start 40.64 86.36) (end 40.64 109.22) (width 0) (layer "B.Cu") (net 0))
 (segment (start 175.26 35.56) (end 83.82 35.56) (width 0.25) (layer "B.Cu") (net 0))
 (segment (start 177.8 38.1) (end 175.26 35.56) (width 0.25) (layer "B.Cu") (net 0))
 (segment (start 27.86 83.86) (end 38.14 83.86) (width 0) (layer "B.Cu") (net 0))
 (segment (start 17.78 127) (end 17.78 130.3) (width 0) (layer "B.Cu") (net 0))
 (segment (start 83.82 20.32) (end 83.82 33.02) (width 0.25) (layer "B.Cu") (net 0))
 (segment (start 35.56 132.08) (end 22.86 132.08) (width 0) (layer "B.Cu") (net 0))
 (segment (start 94.02 134.58) (end 99.06 129.54) (width 0) (layer "B.Cu") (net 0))
 (segment (start 78.74 106.68) (end 78.74 109.22) (width 0) (layer "B.Cu") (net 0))
 (segment (start 83.82 33.02) (end 81.28 35.56) (width 0.25) (layer "B.Cu") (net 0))
 (segment (start 25.4 131.24) (end 19.56 137.08) (width 0) (layer "B.Cu") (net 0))
 (segment (start 96.52 109.22) (end 96.52 66.04) (width 0) (layer "B.Cu") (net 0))
 (segment (start 129.54 99.06) (end 129.54 68.58) (width 0) (layer "B.Cu") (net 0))
 (segment (start 25.4 63.5) (end 33.02 63.5) (width 0) (layer "B.Cu") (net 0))
 (segment (start 22.86 121.92) (end 17.78 127) (width 0) (layer "B.Cu") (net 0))
 (segment (start 81.28 35.56) (end 40.64 35.56) (width 0.25) (layer "B.Cu") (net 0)))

